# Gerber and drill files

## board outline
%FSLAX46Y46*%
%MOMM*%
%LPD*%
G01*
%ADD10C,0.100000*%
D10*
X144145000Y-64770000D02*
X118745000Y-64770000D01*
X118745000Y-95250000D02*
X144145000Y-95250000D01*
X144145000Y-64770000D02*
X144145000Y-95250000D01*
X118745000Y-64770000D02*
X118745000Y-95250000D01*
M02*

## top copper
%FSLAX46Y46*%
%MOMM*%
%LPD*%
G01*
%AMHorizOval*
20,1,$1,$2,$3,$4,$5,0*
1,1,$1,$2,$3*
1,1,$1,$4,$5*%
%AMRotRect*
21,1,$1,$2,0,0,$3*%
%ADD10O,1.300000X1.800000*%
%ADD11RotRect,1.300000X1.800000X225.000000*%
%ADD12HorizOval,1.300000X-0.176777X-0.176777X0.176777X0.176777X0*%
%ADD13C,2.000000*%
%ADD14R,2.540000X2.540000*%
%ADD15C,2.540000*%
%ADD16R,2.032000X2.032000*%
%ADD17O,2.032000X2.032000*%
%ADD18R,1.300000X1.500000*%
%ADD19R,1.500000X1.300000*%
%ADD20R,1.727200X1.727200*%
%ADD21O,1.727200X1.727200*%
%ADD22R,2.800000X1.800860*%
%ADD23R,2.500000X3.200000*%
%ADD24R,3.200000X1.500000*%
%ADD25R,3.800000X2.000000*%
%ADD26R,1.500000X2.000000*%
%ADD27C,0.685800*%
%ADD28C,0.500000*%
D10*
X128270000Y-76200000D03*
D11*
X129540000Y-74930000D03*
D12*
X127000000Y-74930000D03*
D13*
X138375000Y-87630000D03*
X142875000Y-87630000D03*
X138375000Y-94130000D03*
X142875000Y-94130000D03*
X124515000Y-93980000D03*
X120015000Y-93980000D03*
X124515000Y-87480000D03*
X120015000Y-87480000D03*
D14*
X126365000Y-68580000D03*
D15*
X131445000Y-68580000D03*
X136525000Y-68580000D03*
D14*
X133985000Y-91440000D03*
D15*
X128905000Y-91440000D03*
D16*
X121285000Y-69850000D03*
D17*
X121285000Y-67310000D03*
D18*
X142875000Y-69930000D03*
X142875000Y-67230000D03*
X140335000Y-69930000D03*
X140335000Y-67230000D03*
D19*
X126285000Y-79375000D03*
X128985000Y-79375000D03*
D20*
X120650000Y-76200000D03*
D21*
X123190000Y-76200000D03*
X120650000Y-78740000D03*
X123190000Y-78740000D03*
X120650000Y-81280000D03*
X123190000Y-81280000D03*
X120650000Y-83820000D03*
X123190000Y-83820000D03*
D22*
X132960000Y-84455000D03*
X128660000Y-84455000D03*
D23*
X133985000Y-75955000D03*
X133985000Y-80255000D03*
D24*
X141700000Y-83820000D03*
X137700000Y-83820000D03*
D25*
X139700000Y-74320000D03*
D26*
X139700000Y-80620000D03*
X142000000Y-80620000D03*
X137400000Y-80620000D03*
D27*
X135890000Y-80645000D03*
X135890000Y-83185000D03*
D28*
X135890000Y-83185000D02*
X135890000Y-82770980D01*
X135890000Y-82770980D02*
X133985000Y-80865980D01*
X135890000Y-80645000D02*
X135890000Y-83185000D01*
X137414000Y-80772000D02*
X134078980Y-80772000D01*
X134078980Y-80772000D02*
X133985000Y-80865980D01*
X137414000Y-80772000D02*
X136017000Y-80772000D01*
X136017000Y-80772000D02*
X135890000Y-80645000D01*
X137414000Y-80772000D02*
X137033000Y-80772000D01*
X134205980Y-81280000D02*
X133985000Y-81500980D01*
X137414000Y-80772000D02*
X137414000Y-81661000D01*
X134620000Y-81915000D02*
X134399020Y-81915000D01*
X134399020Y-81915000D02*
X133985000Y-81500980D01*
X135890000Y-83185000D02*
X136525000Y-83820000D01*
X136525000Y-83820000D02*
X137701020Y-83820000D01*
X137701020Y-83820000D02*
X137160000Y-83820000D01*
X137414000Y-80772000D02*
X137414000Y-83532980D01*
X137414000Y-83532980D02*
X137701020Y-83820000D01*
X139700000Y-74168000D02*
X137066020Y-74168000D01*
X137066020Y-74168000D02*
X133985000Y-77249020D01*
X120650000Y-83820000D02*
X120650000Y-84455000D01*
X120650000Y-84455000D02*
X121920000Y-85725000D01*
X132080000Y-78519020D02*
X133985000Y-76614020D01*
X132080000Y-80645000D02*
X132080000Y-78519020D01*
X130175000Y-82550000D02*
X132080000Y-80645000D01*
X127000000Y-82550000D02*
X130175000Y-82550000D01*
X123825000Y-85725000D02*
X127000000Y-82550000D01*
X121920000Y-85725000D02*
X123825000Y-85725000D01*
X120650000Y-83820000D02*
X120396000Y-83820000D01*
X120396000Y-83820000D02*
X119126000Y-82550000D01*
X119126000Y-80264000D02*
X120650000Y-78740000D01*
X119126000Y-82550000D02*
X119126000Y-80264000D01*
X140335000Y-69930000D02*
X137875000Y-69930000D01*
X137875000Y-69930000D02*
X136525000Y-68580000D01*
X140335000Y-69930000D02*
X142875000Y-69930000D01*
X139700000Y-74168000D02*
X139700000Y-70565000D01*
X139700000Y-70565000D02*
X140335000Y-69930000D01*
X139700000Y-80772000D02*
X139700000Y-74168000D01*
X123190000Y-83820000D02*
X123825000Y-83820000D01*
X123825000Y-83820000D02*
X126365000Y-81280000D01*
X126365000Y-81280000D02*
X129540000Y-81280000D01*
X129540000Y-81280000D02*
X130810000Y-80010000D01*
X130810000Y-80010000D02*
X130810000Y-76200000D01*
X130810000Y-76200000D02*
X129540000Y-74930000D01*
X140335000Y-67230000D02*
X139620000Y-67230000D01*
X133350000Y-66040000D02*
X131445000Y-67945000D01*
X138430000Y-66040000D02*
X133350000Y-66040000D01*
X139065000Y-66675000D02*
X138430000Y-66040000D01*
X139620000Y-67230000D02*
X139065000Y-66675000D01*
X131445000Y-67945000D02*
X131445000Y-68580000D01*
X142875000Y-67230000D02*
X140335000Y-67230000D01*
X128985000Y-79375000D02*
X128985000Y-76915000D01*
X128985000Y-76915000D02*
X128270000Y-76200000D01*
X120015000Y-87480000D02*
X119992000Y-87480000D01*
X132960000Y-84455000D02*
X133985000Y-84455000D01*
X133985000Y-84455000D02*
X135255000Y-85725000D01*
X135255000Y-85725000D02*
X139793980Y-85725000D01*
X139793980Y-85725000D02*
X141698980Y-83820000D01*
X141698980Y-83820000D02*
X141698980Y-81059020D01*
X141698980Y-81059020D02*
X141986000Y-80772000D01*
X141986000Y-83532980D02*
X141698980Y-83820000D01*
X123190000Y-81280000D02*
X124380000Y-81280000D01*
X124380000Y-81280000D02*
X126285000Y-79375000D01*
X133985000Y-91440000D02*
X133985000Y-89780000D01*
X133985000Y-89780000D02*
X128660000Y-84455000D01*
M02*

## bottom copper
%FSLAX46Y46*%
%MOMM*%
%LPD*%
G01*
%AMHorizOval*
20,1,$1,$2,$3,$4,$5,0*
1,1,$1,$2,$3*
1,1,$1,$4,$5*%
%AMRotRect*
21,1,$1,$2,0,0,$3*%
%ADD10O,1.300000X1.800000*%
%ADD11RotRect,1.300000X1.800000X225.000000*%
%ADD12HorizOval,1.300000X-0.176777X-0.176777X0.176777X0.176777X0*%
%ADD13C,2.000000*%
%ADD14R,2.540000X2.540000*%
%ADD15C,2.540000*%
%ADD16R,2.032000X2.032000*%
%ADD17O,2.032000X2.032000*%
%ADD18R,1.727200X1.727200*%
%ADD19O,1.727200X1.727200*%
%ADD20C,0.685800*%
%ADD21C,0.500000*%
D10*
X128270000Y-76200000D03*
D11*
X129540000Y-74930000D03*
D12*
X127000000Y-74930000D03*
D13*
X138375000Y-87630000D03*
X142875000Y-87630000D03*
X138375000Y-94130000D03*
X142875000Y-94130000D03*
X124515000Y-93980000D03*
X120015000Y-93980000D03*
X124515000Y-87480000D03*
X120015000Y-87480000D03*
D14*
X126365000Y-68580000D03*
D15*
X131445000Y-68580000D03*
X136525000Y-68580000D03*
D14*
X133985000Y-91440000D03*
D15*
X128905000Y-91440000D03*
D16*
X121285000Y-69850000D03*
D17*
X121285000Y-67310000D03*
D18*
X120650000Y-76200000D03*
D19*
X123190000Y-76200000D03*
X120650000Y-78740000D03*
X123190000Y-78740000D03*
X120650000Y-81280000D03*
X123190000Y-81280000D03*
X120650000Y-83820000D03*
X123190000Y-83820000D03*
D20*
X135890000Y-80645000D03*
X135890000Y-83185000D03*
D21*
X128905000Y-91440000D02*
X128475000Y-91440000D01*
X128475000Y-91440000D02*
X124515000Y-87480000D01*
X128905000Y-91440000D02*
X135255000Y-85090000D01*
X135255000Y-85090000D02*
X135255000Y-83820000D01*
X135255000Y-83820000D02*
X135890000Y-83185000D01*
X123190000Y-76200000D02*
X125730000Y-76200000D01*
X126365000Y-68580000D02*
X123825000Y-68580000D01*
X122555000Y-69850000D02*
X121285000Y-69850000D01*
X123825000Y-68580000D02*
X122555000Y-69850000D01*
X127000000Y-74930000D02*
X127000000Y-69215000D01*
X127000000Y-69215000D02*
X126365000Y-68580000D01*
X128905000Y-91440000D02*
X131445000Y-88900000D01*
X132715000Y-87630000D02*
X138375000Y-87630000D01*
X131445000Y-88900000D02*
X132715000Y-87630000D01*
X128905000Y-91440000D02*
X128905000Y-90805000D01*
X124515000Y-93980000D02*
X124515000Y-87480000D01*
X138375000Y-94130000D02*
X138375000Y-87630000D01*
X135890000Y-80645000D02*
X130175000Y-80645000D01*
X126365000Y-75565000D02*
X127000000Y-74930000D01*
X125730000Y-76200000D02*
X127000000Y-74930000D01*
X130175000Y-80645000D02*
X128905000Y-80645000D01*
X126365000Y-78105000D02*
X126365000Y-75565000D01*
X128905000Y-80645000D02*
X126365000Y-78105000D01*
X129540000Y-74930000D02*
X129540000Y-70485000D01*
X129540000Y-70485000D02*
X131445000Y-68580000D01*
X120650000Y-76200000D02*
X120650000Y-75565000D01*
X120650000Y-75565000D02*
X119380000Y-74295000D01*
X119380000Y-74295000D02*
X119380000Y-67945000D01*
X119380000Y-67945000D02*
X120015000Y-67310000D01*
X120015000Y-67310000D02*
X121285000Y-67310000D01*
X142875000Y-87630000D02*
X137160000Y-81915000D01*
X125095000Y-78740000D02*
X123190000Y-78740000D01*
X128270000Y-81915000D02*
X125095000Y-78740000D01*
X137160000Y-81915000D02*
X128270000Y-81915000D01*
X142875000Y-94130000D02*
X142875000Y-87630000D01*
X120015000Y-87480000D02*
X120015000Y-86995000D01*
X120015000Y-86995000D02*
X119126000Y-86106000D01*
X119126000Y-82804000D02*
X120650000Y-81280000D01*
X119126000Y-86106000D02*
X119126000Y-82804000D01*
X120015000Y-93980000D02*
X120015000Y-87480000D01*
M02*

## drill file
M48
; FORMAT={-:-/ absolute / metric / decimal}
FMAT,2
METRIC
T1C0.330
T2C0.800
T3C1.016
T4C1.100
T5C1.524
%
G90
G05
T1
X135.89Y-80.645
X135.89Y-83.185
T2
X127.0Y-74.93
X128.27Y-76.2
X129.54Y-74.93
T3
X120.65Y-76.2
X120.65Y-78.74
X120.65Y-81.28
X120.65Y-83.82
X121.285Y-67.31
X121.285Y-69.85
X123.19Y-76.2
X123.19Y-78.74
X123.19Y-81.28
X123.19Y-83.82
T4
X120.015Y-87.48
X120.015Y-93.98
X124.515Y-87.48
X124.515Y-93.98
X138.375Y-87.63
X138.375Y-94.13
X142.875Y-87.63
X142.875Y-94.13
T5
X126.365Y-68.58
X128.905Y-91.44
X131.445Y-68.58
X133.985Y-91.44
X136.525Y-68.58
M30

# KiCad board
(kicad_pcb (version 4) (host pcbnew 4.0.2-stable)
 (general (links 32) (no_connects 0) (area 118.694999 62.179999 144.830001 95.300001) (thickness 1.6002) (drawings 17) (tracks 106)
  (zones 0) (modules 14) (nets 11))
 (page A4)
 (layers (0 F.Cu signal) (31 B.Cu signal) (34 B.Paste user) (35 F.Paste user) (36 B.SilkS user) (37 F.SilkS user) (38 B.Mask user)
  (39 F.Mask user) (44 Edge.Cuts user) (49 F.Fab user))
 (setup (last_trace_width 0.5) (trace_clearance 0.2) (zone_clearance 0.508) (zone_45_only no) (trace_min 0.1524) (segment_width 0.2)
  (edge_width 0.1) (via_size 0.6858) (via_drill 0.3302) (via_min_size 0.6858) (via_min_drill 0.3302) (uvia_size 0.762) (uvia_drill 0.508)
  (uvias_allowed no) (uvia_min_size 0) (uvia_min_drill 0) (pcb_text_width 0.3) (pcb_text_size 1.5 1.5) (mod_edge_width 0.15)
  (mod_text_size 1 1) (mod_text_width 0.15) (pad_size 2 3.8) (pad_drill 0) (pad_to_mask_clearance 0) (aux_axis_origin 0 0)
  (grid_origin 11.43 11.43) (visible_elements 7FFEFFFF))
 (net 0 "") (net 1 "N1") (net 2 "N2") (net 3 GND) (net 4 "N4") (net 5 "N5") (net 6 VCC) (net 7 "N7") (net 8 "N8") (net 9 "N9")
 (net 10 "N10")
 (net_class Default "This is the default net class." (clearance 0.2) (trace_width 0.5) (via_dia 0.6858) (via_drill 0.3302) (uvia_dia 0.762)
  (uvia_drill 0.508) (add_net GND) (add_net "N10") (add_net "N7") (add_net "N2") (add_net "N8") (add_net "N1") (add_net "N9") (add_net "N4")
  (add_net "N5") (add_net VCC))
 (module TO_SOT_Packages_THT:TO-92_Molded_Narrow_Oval (layer F.Cu) (at 129.54 74.93 180)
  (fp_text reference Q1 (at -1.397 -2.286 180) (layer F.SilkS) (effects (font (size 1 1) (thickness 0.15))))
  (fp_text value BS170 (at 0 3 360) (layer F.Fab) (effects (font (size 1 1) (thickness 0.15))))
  (pad 2 thru_hole oval (at 1.27 -1.27 270) (size 1.8 1.3) (drill 0.8) (layers *.Cu *.Mask) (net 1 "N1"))
  (pad 1 thru_hole rect (at 0 0 225) (size 1.3 1.8) (drill 0.8) (layers *.Cu *.Mask) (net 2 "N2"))
  (pad 3 thru_hole oval (at 2.54 0 225) (size 1.8 1.3) (drill 0.8) (layers *.Cu *.Mask) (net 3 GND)))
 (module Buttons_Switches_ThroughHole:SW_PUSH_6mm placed (layer F.Cu) (at 142.875 87.63 270)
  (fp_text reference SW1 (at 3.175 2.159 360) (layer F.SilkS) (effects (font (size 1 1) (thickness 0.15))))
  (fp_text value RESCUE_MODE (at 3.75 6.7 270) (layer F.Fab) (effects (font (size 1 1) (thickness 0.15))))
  (pad 2 thru_hole circle (at 0 4.5) (size 2 2) (drill 1.1) (layers *.Cu *.Mask) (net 3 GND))
  (pad 1 thru_hole circle (at 0 0) (size 2 2) (drill 1.1) (layers *.Cu *.Mask) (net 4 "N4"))
  (pad 2 thru_hole circle (at 6.5 4.5) (size 2 2) (drill 1.1) (layers *.Cu *.Mask) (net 3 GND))
  (pad 1 thru_hole circle (at 6.5 0) (size 2 2) (drill 1.1) (layers *.Cu *.Mask) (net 4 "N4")))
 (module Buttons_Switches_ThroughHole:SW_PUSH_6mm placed (layer F.Cu) (at 120.015 93.98 90)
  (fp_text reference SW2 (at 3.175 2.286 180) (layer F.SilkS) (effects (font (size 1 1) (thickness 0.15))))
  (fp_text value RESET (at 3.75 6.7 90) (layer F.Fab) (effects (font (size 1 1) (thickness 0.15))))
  (pad 2 thru_hole circle (at 0 4.5 180) (size 2 2) (drill 1.1) (layers *.Cu *.Mask) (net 3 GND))
  (pad 1 thru_hole circle (at 0 0 180) (size 2 2) (drill 1.1) (layers *.Cu *.Mask) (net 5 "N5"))
  (pad 2 thru_hole circle (at 6.5 4.5 180) (size 2 2) (drill 1.1) (layers *.Cu *.Mask) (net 3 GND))
  (pad 1 thru_hole circle (at 6.5 0 180) (size 2 2) (drill 1.1) (layers *.Cu *.Mask) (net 5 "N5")))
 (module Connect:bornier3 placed (layer F.Cu) (at 131.445 68.58)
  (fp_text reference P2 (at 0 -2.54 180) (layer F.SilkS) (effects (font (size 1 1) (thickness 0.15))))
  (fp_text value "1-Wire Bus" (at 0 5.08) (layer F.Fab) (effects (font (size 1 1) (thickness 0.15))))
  (pad 1 thru_hole rect (at -5.08 0) (size 2.54 2.54) (drill 1.524) (layers *.Cu *.Mask F.SilkS) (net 3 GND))
  (pad 2 thru_hole circle (at 0 0) (size 2.54 2.54) (drill 1.524) (layers *.Cu *.Mask F.SilkS) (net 2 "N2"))
  (pad 3 thru_hole circle (at 5.08 0) (size 2.54 2.54) (drill 1.524) (layers *.Cu *.Mask F.SilkS) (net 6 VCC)))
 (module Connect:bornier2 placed (layer F.Cu) (at 131.445 91.44 180)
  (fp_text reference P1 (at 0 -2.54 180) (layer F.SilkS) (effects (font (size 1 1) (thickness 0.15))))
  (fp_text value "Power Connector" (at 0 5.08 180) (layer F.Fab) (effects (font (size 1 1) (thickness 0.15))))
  (pad 1 thru_hole rect (at -2.54 0 180) (size 2.54 2.54) (drill 1.524) (layers *.Cu *.Mask F.SilkS) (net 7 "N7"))
  (pad 2 thru_hole circle (at 2.54 0 180) (size 2.54 2.54) (drill 1.524) (layers *.Cu *.Mask F.SilkS) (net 3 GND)))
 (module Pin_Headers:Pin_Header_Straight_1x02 (layer F.Cu) (at 121.285 69.85 180)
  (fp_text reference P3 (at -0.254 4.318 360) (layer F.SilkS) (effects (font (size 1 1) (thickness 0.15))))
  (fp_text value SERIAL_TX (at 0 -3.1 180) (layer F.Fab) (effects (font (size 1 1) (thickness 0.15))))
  (pad 1 thru_hole rect (at 0 0 180) (size 2.032 2.032) (drill 1.016) (layers *.Cu *.Mask F.SilkS) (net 3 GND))
  (pad 2 thru_hole oval (at 0 2.54 180) (size 2.032 2.032) (drill 1.016) (layers *.Cu *.Mask F.SilkS) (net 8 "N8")))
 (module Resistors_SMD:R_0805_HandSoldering (layer F.Cu) (at 142.875 68.58 90)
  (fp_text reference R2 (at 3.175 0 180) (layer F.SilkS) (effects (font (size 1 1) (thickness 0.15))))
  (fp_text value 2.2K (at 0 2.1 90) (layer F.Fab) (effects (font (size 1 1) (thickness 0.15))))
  (pad 1 smd rect (at -1.35 0 90) (size 1.5 1.3) (layers F.Cu F.Paste F.Mask) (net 6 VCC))
  (pad 2 smd rect (at 1.35 0 90) (size 1.5 1.3) (layers F.Cu F.Paste F.Mask) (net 2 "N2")))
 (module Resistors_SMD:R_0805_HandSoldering (layer F.Cu) (at 140.335 68.58 90)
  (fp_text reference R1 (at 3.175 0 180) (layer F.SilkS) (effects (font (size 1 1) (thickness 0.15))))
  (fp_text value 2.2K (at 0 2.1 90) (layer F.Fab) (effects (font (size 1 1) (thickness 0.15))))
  (pad 1 smd rect (at -1.35 0 90) (size 1.5 1.3) (layers F.Cu F.Paste F.Mask) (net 6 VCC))
  (pad 2 smd rect (at 1.35 0 90) (size 1.5 1.3) (layers F.Cu F.Paste F.Mask) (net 2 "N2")))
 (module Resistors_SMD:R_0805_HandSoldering (layer F.Cu) (at 127.635 79.375)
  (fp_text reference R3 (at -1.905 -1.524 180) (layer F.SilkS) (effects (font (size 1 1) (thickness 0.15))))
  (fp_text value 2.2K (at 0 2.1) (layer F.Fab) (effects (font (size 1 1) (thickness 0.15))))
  (pad 1 smd rect (at -1.35 0) (size 1.5 1.3) (layers F.Cu F.Paste F.Mask) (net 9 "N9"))
  (pad 2 smd rect (at 1.35 0) (size 1.5 1.3) (layers F.Cu F.Paste F.Mask) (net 1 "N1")))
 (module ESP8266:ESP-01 (layer F.Cu) (at 120.65 76.2)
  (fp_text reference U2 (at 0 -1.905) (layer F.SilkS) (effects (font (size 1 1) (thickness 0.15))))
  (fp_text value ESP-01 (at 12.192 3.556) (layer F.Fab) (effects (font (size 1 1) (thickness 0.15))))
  (pad 1 thru_hole rect (at 0 0) (size 1.7272 1.7272) (drill 1.016) (layers *.Cu *.Mask F.SilkS) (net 8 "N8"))
  (pad 2 thru_hole oval (at 2.54 0) (size 1.7272 1.7272) (drill 1.016) (layers *.Cu *.Mask F.SilkS) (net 3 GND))
  (pad 3 thru_hole oval (at 0 2.54) (size 1.7272 1.7272) (drill 1.016) (layers *.Cu *.Mask F.SilkS) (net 6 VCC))
  (pad 4 thru_hole oval (at 2.54 2.54) (size 1.7272 1.7272) (drill 1.016) (layers *.Cu *.Mask F.SilkS) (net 4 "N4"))
  (pad 5 thru_hole oval (at 0 5.08) (size 1.7272 1.7272) (drill 1.016) (layers *.Cu *.Mask F.SilkS) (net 5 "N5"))
  (pad 6 thru_hole oval (at 2.54 5.08) (size 1.7272 1.7272) (drill 1.016) (layers *.Cu *.Mask F.SilkS) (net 9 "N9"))
  (pad 7 thru_hole oval (at 0 7.62) (size 1.7272 1.7272) (drill 1.016) (layers *.Cu *.Mask F.SilkS) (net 6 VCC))
  (pad 8 thru_hole oval (at 2.54 7.62) (size 1.7272 1.7272) (drill 1.016) (layers *.Cu *.Mask F.SilkS) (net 2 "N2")))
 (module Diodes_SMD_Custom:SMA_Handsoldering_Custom (layer F.Cu) (at 130.81 84.455 180)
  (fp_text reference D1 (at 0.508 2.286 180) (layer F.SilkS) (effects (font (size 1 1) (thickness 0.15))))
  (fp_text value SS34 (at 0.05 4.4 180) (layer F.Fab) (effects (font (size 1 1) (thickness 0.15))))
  (pad 1 smd rect (at -2.15 0 180) (size 2.8 1.80086) (layers F.Cu F.Paste F.Mask) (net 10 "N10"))
  (pad 2 smd rect (at 2.15 0 180) (size 2.8 1.80086) (layers F.Cu F.Paste F.Mask) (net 7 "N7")))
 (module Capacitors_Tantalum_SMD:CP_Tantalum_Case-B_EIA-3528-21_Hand (layer F.Cu) (at 133.985 78.105 270)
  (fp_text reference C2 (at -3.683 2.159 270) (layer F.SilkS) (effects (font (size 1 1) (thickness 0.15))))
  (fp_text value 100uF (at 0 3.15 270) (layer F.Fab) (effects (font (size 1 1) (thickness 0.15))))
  (pad 1 smd rect (at -2.15 0 270) (size 3.2 2.5) (layers F.Cu F.Paste F.Mask) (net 6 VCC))
  (pad 2 smd rect (at 2.15 0 270) (size 3.2 2.5) (layers F.Cu F.Paste F.Mask) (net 3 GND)))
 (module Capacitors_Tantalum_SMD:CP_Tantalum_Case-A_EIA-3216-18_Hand (layer F.Cu) (at 139.7 83.82 180)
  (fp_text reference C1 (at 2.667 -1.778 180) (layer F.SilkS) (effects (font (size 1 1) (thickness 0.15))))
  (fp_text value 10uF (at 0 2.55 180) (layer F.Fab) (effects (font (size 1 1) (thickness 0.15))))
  (pad 1 smd rect (at -2 0 180) (size 3.2 1.5) (layers F.Cu F.Paste F.Mask) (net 10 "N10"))
  (pad 2 smd rect (at 2 0 180) (size 3.2 1.5) (layers F.Cu F.Paste F.Mask) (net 3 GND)))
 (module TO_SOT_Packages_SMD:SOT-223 (layer F.Cu) (at 139.7 77.47 90)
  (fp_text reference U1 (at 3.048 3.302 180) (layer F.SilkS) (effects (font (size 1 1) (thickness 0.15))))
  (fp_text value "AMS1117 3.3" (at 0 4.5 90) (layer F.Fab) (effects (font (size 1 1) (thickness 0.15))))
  (pad 4 smd rect (at 3.15 0 90) (size 2 3.8) (layers F.Cu F.Paste F.Mask) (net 6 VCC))
  (pad 2 smd rect (at -3.15 0 90) (size 2 1.5) (layers F.Cu F.Paste F.Mask) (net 6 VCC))
  (pad 3 smd rect (at -3.15 2.3 90) (size 2 1.5) (layers F.Cu F.Paste F.Mask) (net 10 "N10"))
  (pad 1 smd rect (at -3.15 -2.3 90) (size 2 1.5) (layers F.Cu F.Paste F.Mask) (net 3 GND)))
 (gr_line (start 144.145 64.77) (end 118.745 64.77) (angle 90) (layer Edge.Cuts) (width 0.1))
 (gr_line (start 118.745 95.25) (end 144.145 95.25) (angle 90) (layer Edge.Cuts) (width 0.1))
 (gr_line (start 144.145 64.77) (end 144.145 95.25) (angle 90) (layer Edge.Cuts) (width 0.1))
 (gr_line (start 118.745 64.77) (end 118.745 95.25) (angle 90) (layer Edge.Cuts) (width 0.1))
 (segment (start 135.89 83.185) (end 135.89 82.77098) (width 0.5) (layer F.Cu) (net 3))
 (segment (start 135.89 82.77098) (end 133.985 80.86598) (width 0.5) (layer F.Cu) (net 3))
 (segment (start 135.89 80.645) (end 135.89 83.185) (width 0.5) (layer F.Cu) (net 3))
 (segment (start 137.414 80.772) (end 134.07898 80.772) (width 0.5) (layer F.Cu) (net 3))
 (segment (start 134.07898 80.772) (end 133.985 80.86598) (width 0.5) (layer F.Cu) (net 3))
 (segment (start 128.905 91.44) (end 128.475 91.44) (width 0.5) (layer B.Cu) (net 3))
 (segment (start 128.475 91.44) (end 124.515 87.48) (width 0.5) (layer B.Cu) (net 3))
 (segment (start 137.414 80.772) (end 136.017 80.772) (width 0.5) (layer F.Cu) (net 3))
 (via (at 135.89 80.645) (size 0.6858) (drill 0.3302) (layers F.Cu B.Cu) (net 3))
 (segment (start 136.017 80.772) (end 135.89 80.645) (width 0.5) (layer F.Cu) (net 3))
 (segment (start 137.414 80.772) (end 137.033 80.772) (width 0.5) (layer F.Cu) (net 3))
 (segment (start 134.20598 81.28) (end 133.985 81.50098) (width 0.5) (layer F.Cu) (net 3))
 (segment (start 137.414 80.772) (end 137.414 81.661) (width 0.5) (layer F.Cu) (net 3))
 (segment (start 134.62 81.915) (end 134.39902 81.915) (width 0.5) (layer F.Cu) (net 3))
 (segment (start 134.39902 81.915) (end 133.985 81.50098) (width 0.5) (layer F.Cu) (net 3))
 (segment (start 128.905 91.44) (end 135.255 85.09) (width 0.5) (layer B.Cu) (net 3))
 (segment (start 135.255 85.09) (end 135.255 83.82) (width 0.5) (layer B.Cu) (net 3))
 (segment (start 135.255 83.82) (end 135.89 83.185) (width 0.5) (layer B.Cu) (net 3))
 (via (at 135.89 83.185) (size 0.6858) (drill 0.3302) (layers F.Cu B.Cu) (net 3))
 (segment (start 135.89 83.185) (end 136.525 83.82) (width 0.5) (layer F.Cu) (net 3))
 (segment (start 136.525 83.82) (end 137.70102 83.82) (width 0.5) (layer F.Cu) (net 3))
 (segment (start 123.19 76.2) (end 125.73 76.2) (width 0.5) (layer B.Cu) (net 3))
 (segment (start 126.365 68.58) (end 123.825 68.58) (width 0.5) (layer B.Cu) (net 3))
 (segment (start 122.555 69.85) (end 121.285 69.85) (width 0.5) (layer B.Cu) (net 3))
 (segment (start 123.825 68.58) (end 122.555 69.85) (width 0.5) (layer B.Cu) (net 3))
 (segment (start 127 74.93) (end 127 69.215) (width 0.5) (layer B.Cu) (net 3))
 (segment (start 127 69.215) (end 126.365 68.58) (width 0.5) (layer B.Cu) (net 3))
 (segment (start 137.70102 83.82) (end 137.16 83.82) (width 0.5) (layer F.Cu) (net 3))
 (segment (start 128.905 91.44) (end 131.445 88.9) (width 0.5) (layer B.Cu) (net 3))
 (segment (start 132.715 87.63) (end 138.375 87.63) (width 0.5) (layer B.Cu) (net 3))
 (segment (start 131.445 88.9) (end 132.715 87.63) (width 0.5) (layer B.Cu) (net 3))
 (segment (start 128.905 91.44) (end 128.905 90.805) (width 0.5) (layer B.Cu) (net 3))
 (segment (start 137.414 80.772) (end 137.414 83.53298) (width 0.5) (layer F.Cu) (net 3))
 (segment (start 137.414 83.53298) (end 137.70102 83.82) (width 0.5) (layer F.Cu) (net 3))
 (segment (start 124.515 93.98) (end 124.515 87.48) (width 0.5) (layer B.Cu) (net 3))
 (segment (start 138.375 94.13) (end 138.375 87.63) (width 0.5) (layer B.Cu) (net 3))
 (segment (start 135.89 80.645) (end 130.175 80.645) (width 0.5) (layer B.Cu) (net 3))
 (segment (start 126.365 75.565) (end 127 74.93) (width 0.5) (layer B.Cu) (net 3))
 (segment (start 125.73 76.2) (end 127 74.93) (width 0.5) (layer B.Cu) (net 3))
 (segment (start 130.175 80.645) (end 128.905 80.645) (width 0.5) (layer B.Cu) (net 3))
 (segment (start 126.365 78.105) (end 126.365 75.565) (width 0.5) (layer B.Cu) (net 3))
 (segment (start 128.905 80.645) (end 126.365 78.105) (width 0.5) (layer B.Cu) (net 3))
 (segment (start 139.7 74.168) (end 137.06602 74.168) (width 0.5) (layer F.Cu) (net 6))
 (segment (start 137.06602 74.168) (end 133.985 77.24902) (width 0.5) (layer F.Cu) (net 6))
 (segment (start 120.65 83.82) (end 120.65 84.455) (width 0.5) (layer F.Cu) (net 6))
 (segment (start 120.65 84.455) (end 121.92 85.725) (width 0.5) (layer F.Cu) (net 6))
 (segment (start 132.08 78.51902) (end 133.985 76.61402) (width 0.5) (layer F.Cu) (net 6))
 (segment (start 132.08 80.645) (end 132.08 78.51902) (width 0.5) (layer F.Cu) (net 6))
 (segment (start 130.175 82.55) (end 132.08 80.645) (width 0.5) (layer F.Cu) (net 6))
 (segment (start 127 82.55) (end 130.175 82.55) (width 0.5) (layer F.Cu) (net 6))
 (segment (start 123.825 85.725) (end 127 82.55) (width 0.5) (layer F.Cu) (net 6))
 (segment (start 121.92 85.725) (end 123.825 85.725) (width 0.5) (layer F.Cu) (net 6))
 (segment (start 120.65 83.82) (end 120.396 83.82) (width 0.5) (layer F.Cu) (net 6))
 (segment (start 120.396 83.82) (end 119.126 82.55) (width 0.5) (layer F.Cu) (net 6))
 (segment (start 119.126 80.264) (end 120.65 78.74) (width 0.5) (layer F.Cu) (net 6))
 (segment (start 119.126 82.55) (end 119.126 80.264) (width 0.5) (layer F.Cu) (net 6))
 (segment (start 140.335 69.93) (end 137.875 69.93) (width 0.5) (layer F.Cu) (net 6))
 (segment (start 137.875 69.93) (end 136.525 68.58) (width 0.5) (layer F.Cu) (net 6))
 (segment (start 140.335 69.93) (end 142.875 69.93) (width 0.5) (layer F.Cu) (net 6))
 (segment (start 139.7 74.168) (end 139.7 70.565) (width 0.5) (layer F.Cu) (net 6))
 (segment (start 139.7 70.565) (end 140.335 69.93) (width 0.5) (layer F.Cu) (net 6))
 (segment (start 139.7 80.772) (end 139.7 74.168) (width 0.5) (layer F.Cu) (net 6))
 (segment (start 123.19 83.82) (end 123.825 83.82) (width 0.5) (layer F.Cu) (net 2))
 (segment (start 123.825 83.82) (end 126.365 81.28) (width 0.5) (layer F.Cu) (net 2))
 (segment (start 126.365 81.28) (end 129.54 81.28) (width 0.5) (layer F.Cu) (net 2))
 (segment (start 129.54 81.28) (end 130.81 80.01) (width 0.5) (layer F.Cu) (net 2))
 (segment (start 130.81 80.01) (end 130.81 76.2) (width 0.5) (layer F.Cu) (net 2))
 (segment (start 130.81 76.2) (end 129.54 74.93) (width 0.5) (layer F.Cu) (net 2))
 (segment (start 129.54 74.93) (end 129.54 70.485) (width 0.5) (layer B.Cu) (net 2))
 (segment (start 129.54 70.485) (end 131.445 68.58) (width 0.5) (layer B.Cu) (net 2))
 (segment (start 140.335 67.23) (end 139.62 67.23) (width 0.5) (layer F.Cu) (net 2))
 (segment (start 133.35 66.04) (end 131.445 67.945) (width 0.5) (layer F.Cu) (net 2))
 (segment (start 138.43 66.04) (end 133.35 66.04) (width 0.5) (layer F.Cu) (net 2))
 (segment (start 139.065 66.675) (end 138.43 66.04) (width 0.5) (layer F.Cu) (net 2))
 (segment (start 139.62 67.23) (end 139.065 66.675) (width 0.5) (layer F.Cu) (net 2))
 (segment (start 131.445 67.945) (end 131.445 68.58) (width 0.5) (layer F.Cu) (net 2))
 (segment (start 142.875 67.23) (end 140.335 67.23) (width 0.5) (layer F.Cu) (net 2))
 (segment (start 120.65 76.2) (end 120.65 75.565) (width 0.5) (layer B.Cu) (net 8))
 (segment (start 120.65 75.565) (end 119.38 74.295) (width 0.5) (layer B.Cu) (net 8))
 (segment (start 119.38 74.295) (end 119.38 67.945) (width 0.5) (layer B.Cu) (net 8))
 (segment (start 119.38 67.945) (end 120.015 67.31) (width 0.5) (layer B.Cu) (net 8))
 (segment (start 120.015 67.31) (end 121.285 67.31) (width 0.5) (layer B.Cu) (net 8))
 (segment (start 128.985 79.375) (end 128.985 76.915) (width 0.5) (layer F.Cu) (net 1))
 (segment (start 128.985 76.915) (end 128.27 76.2) (width 0.5) (layer F.Cu) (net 1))
 (segment (start 142.875 87.63) (end 137.16 81.915) (width 0.5) (layer B.Cu) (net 4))
 (segment (start 125.095 78.74) (end 123.19 78.74) (width 0.5) (layer B.Cu) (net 4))
 (segment (start 128.27 81.915) (end 125.095 78.74) (width 0.5) (layer B.Cu) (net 4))
 (segment (start 137.16 81.915) (end 128.27 81.915) (width 0.5) (layer B.Cu) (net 4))
 (segment (start 142.875 94.13) (end 142.875 87.63) (width 0.5) (layer B.Cu) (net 4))
 (segment (start 120.015 87.48) (end 120.015 86.995) (width 0.5) (layer B.Cu) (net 5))
 (segment (start 120.015 86.995) (end 119.126 86.106) (width 0.5) (layer B.Cu) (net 5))
 (segment (start 119.126 82.804) (end 120.65 81.28) (width 0.5) (layer B.Cu) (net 5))
 (segment (start 119.126 86.106) (end 119.126 82.804) (width 0.5) (layer B.Cu) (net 5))
 (segment (start 120.015 87.48) (end 119.992 87.48) (width 0.5) (layer F.Cu) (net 5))
 (segment (start 120.015 93.98) (end 120.015 87.48) (width 0.5) (layer B.Cu) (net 5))
 (segment (start 132.96 84.455) (end 133.985 84.455) (width 0.5) (layer F.Cu) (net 10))
 (segment (start 133.985 84.455) (end 135.255 85.725) (width 0.5) (layer F.Cu) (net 10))
 (segment (start 135.255 85.725) (end 139.79398 85.725) (width 0.5) (layer F.Cu) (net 10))
 (segment (start 139.79398 85.725) (end 141.69898 83.82) (width 0.5) (layer F.Cu) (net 10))
 (segment (start 141.69898 83.82) (end 141.69898 81.05902) (width 0.5) (layer F.Cu) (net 10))
 (segment (start 141.69898 81.05902) (end 141.986 80.772) (width 0.5) (layer F.Cu) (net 10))
 (segment (start 141.986 83.53298) (end 141.69898 83.82) (width 0.5) (layer F.Cu) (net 10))
 (segment (start 123.19 81.28) (end 124.38 81.28) (width 0.5) (layer F.Cu) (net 9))
 (segment (start 124.38 81.28) (end 126.285 79.375) (width 0.5) (layer F.Cu) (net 9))
 (segment (start 133.985 91.44) (end 133.985 89.78) (width 0.5) (layer F.Cu) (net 7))
 (segment (start 133.985 89.78) (end 128.66 84.455) (width 0.5) (layer F.Cu) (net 7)))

